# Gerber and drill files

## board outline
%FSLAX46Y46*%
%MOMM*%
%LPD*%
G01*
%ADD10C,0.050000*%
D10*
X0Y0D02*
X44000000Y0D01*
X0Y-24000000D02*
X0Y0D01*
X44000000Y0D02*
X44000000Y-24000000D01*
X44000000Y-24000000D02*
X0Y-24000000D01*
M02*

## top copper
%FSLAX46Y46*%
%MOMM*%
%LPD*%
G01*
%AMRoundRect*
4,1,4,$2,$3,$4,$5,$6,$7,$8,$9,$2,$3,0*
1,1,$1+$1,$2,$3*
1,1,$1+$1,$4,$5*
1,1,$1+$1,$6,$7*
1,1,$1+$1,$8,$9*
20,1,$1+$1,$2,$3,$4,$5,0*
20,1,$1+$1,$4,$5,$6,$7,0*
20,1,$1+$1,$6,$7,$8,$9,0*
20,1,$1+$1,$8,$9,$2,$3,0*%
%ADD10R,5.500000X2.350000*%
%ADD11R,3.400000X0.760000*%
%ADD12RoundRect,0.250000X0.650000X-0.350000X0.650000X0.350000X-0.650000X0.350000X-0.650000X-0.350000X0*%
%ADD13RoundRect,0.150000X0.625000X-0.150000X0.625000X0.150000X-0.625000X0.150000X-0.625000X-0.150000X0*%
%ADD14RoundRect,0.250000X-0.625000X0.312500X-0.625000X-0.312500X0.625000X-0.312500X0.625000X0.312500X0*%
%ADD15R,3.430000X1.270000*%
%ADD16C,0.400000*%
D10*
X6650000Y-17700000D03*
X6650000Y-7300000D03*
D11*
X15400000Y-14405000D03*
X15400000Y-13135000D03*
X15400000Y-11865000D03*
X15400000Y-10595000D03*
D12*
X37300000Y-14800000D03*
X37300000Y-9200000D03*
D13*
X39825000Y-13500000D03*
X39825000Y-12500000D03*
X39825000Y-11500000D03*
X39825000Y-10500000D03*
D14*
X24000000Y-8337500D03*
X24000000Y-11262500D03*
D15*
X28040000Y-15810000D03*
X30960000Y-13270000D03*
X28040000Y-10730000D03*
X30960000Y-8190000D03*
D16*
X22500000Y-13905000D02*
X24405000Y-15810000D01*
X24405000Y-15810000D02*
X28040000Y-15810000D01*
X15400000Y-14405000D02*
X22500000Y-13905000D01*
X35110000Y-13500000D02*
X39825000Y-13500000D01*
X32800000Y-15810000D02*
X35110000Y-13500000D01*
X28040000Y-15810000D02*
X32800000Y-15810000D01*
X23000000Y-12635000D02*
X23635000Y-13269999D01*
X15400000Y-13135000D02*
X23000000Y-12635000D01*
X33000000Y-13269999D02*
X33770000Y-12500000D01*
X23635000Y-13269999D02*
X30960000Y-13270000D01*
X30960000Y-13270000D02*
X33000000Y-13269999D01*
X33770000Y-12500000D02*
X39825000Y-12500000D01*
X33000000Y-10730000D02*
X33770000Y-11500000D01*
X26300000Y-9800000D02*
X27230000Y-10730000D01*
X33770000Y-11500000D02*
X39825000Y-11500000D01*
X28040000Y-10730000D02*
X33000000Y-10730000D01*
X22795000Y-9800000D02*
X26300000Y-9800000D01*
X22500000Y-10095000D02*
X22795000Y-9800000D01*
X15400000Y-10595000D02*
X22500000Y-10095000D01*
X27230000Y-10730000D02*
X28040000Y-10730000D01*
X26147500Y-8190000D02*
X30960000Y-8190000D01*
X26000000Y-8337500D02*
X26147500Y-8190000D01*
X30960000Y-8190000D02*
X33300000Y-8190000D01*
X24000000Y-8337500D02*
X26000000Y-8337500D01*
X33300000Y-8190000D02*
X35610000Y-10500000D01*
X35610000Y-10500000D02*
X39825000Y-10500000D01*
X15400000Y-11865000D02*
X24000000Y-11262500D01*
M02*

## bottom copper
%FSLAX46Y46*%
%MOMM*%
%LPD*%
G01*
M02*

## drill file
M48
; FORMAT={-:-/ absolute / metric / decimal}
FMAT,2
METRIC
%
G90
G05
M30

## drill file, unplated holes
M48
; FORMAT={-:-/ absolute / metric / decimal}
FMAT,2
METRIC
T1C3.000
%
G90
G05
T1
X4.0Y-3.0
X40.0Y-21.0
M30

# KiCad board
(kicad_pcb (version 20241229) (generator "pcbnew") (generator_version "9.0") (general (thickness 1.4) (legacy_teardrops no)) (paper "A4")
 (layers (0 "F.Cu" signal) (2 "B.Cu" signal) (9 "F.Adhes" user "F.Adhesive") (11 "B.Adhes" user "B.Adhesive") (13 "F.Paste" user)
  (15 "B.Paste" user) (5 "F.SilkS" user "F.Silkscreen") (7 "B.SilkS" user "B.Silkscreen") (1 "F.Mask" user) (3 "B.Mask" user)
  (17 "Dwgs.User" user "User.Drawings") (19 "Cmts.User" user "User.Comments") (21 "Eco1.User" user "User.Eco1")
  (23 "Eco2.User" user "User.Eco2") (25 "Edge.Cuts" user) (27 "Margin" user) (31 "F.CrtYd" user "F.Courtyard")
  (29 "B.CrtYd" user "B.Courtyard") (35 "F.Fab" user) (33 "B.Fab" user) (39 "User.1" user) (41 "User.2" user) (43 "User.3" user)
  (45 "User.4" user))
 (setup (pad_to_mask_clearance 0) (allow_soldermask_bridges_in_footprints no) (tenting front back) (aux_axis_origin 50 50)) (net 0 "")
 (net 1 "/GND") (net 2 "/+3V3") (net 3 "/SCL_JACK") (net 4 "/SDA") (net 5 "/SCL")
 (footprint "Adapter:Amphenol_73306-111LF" (layer "F.Cu") (at 51 62.5 90)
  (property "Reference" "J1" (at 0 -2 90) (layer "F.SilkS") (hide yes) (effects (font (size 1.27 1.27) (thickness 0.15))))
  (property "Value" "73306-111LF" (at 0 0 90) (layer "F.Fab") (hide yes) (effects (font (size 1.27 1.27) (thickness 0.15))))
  (pad "" smd rect (at -5.2 5.65 90) (size 2.35 5.5) (layers "F.Cu" "F.Mask" "F.Paste") (thermal_bridge_angle 45))
  (pad "" smd rect (at 5.2 5.65 90) (size 2.35 5.5) (layers "F.Cu" "F.Mask" "F.Paste") (thermal_bridge_angle 45))
  (pad "1" smd rect (at -1.905 14.4 90) (size 0.76 3.4) (layers "F.Cu" "F.Mask" "F.Paste") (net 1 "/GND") (thermal_bridge_angle 45))
  (pad "2" smd rect (at -0.635 14.4 90) (size 0.76 3.4) (layers "F.Cu" "F.Mask" "F.Paste") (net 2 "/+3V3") (thermal_bridge_angle 45))
  (pad "3" smd rect (at 0.635 14.4 90) (size 0.76 3.4) (layers "F.Cu" "F.Mask" "F.Paste") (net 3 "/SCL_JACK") (thermal_bridge_angle 45))
  (pad "4" smd rect (at 1.905 14.4 90) (size 0.76 3.4) (layers "F.Cu" "F.Mask" "F.Paste") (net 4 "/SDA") (thermal_bridge_angle 45)))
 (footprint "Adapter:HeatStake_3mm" (layer "F.Cu") (at 90 71)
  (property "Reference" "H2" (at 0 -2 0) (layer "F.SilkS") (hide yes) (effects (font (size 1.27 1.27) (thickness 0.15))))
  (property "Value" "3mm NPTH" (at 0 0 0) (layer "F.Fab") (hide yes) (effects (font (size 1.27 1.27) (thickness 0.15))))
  (pad "" np_thru_hole circle (at 0 0) (size 3 3) (drill 3) (layers "*.Cu" "*.Mask")))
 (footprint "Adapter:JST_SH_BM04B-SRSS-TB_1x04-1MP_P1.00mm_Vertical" (layer "F.Cu") (at 88.5 62 90)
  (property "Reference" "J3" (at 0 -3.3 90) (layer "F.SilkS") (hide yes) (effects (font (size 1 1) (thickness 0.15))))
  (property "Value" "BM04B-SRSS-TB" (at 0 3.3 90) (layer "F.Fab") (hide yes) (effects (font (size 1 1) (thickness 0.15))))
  (pad "" smd roundrect (at -2.8 -1.2 90) (size 1.2 1.8) (layers "F.Cu" "F.Mask" "F.Paste") (roundrect_rratio 0.208333))
  (pad "" smd roundrect (at 2.8 -1.2 90) (size 1.2 1.8) (layers "F.Cu" "F.Mask" "F.Paste") (roundrect_rratio 0.208333))
  (pad "1" smd roundrect (at -1.5 1.325 90) (size 0.6 1.55) (layers "F.Cu" "F.Mask" "F.Paste") (roundrect_rratio 0.25) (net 1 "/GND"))
  (pad "2" smd roundrect (at -0.5 1.325 90) (size 0.6 1.55) (layers "F.Cu" "F.Mask" "F.Paste") (roundrect_rratio 0.25) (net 2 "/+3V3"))
  (pad "3" smd roundrect (at 0.5 1.325 90) (size 0.6 1.55) (layers "F.Cu" "F.Mask" "F.Paste") (roundrect_rratio 0.25) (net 4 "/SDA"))
  (pad "4" smd roundrect (at 1.5 1.325 90) (size 0.6 1.55) (layers "F.Cu" "F.Mask" "F.Paste") (roundrect_rratio 0.25) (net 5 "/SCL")))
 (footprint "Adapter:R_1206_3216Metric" (layer "F.Cu") (at 74 59.8 -90)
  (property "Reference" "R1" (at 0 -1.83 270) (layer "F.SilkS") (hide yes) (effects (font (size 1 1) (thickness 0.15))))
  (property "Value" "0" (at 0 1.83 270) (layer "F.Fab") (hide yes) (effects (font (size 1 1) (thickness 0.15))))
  (pad "1" smd roundrect (at -1.4625 0 270) (size 1.125 1.75) (layers "F.Cu" "F.Mask" "F.Paste") (roundrect_rratio 0.222222) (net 5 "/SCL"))
  (pad "2" smd roundrect (at 1.4625 0 270) (size 1.125 1.75) (layers "F.Cu" "F.Mask" "F.Paste") (roundrect_rratio 0.222222)
   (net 3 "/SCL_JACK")))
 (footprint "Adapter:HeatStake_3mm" (layer "F.Cu") (at 54 53)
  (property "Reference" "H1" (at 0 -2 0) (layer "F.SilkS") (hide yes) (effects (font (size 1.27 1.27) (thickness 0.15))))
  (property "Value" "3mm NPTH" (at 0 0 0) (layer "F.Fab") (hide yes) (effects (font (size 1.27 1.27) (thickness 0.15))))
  (pad "" np_thru_hole circle (at 0 0) (size 3 3) (drill 3) (layers "*.Cu" "*.Mask")))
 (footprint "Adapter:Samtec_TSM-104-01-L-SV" (layer "F.Cu") (at 79.5 62 -90)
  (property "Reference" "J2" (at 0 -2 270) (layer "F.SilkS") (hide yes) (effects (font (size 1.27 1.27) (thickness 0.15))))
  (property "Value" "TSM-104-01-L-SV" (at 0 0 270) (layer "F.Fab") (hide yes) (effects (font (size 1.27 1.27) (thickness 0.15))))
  (pad "1" smd rect (at 3.81 1.46 270) (size 1.27 3.43) (layers "F.Cu" "F.Mask" "F.Paste") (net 1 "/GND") (thermal_bridge_angle 45))
  (pad "2" smd rect (at 1.27 -1.46 270) (size 1.27 3.43) (layers "F.Cu" "F.Mask" "F.Paste") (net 2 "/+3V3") (thermal_bridge_angle 45))
  (pad "3" smd rect (at -1.27 1.46 270) (size 1.27 3.43) (layers "F.Cu" "F.Mask" "F.Paste") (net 4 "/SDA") (thermal_bridge_angle 45))
  (pad "4" smd rect (at -3.81 -1.46 270) (size 1.27 3.43) (layers "F.Cu" "F.Mask" "F.Paste") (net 5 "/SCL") (thermal_bridge_angle 45)))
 (gr_line (start 50 50) (end 94 50) (stroke (width 0.05) (type default)) (layer "Edge.Cuts"))
 (gr_line (start 50 74) (end 50 50) (stroke (width 0.05) (type default)) (layer "Edge.Cuts"))
 (gr_line (start 94 50) (end 94 74) (stroke (width 0.05) (type default)) (layer "Edge.Cuts"))
 (gr_line (start 94 74) (end 50 74) (stroke (width 0.05) (type default)) (layer "Edge.Cuts"))
 (segment (start 72.5 63.905) (end 74.405 65.81) (width 0.4) (layer "F.Cu") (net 1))
 (segment (start 74.405 65.81) (end 78.04 65.81) (width 0.4) (layer "F.Cu") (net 1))
 (segment (start 65.4 64.405) (end 72.5 63.905) (width 0.4) (layer "F.Cu") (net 1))
 (segment (start 85.11 63.5) (end 89.825 63.5) (width 0.4) (layer "F.Cu") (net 1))
 (segment (start 82.8 65.81) (end 85.11 63.5) (width 0.4) (layer "F.Cu") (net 1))
 (segment (start 78.04 65.81) (end 82.8 65.81) (width 0.4) (layer "F.Cu") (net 1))
 (segment (start 73 62.635) (end 73.635 63.269999) (width 0.4) (layer "F.Cu") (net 2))
 (segment (start 65.4 63.135) (end 73 62.635) (width 0.4) (layer "F.Cu") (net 2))
 (segment (start 83 63.269999) (end 83.77 62.5) (width 0.4) (layer "F.Cu") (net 2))
 (segment (start 73.635 63.269999) (end 80.96 63.27) (width 0.4) (layer "F.Cu") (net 2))
 (segment (start 80.96 63.27) (end 83 63.269999) (width 0.4) (layer "F.Cu") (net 2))
 (segment (start 83.77 62.5) (end 89.825 62.5) (width 0.4) (layer "F.Cu") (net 2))
 (segment (start 83 60.73) (end 83.77 61.5) (width 0.4) (layer "F.Cu") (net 4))
 (segment (start 76.3 59.8) (end 77.23 60.73) (width 0.4) (layer "F.Cu") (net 4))
 (segment (start 83.77 61.5) (end 89.825 61.5) (width 0.4) (layer "F.Cu") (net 4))
 (segment (start 78.04 60.73) (end 83 60.73) (width 0.4) (layer "F.Cu") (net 4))
 (segment (start 72.795 59.8) (end 76.3 59.8) (width 0.4) (layer "F.Cu") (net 4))
 (segment (start 72.5 60.095) (end 72.795 59.8) (width 0.4) (layer "F.Cu") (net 4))
 (segment (start 65.4 60.595) (end 72.5 60.095) (width 0.4) (layer "F.Cu") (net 4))
 (segment (start 77.23 60.73) (end 78.04 60.73) (width 0.4) (layer "F.Cu") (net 4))
 (segment (start 76.1475 58.19) (end 80.96 58.19) (width 0.4) (layer "F.Cu") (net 5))
 (segment (start 76 58.3375) (end 76.1475 58.19) (width 0.4) (layer "F.Cu") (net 5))
 (segment (start 80.96 58.19) (end 83.3 58.19) (width 0.4) (layer "F.Cu") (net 5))
 (segment (start 74 58.3375) (end 76 58.3375) (width 0.4) (layer "F.Cu") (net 5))
 (segment (start 83.3 58.19) (end 85.61 60.5) (width 0.4) (layer "F.Cu") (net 5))
 (segment (start 85.61 60.5) (end 89.825 60.5) (width 0.4) (layer "F.Cu") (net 5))
 (segment (start 65.4 61.865) (end 74 61.2625) (width 0.4) (layer "F.Cu") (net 3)))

